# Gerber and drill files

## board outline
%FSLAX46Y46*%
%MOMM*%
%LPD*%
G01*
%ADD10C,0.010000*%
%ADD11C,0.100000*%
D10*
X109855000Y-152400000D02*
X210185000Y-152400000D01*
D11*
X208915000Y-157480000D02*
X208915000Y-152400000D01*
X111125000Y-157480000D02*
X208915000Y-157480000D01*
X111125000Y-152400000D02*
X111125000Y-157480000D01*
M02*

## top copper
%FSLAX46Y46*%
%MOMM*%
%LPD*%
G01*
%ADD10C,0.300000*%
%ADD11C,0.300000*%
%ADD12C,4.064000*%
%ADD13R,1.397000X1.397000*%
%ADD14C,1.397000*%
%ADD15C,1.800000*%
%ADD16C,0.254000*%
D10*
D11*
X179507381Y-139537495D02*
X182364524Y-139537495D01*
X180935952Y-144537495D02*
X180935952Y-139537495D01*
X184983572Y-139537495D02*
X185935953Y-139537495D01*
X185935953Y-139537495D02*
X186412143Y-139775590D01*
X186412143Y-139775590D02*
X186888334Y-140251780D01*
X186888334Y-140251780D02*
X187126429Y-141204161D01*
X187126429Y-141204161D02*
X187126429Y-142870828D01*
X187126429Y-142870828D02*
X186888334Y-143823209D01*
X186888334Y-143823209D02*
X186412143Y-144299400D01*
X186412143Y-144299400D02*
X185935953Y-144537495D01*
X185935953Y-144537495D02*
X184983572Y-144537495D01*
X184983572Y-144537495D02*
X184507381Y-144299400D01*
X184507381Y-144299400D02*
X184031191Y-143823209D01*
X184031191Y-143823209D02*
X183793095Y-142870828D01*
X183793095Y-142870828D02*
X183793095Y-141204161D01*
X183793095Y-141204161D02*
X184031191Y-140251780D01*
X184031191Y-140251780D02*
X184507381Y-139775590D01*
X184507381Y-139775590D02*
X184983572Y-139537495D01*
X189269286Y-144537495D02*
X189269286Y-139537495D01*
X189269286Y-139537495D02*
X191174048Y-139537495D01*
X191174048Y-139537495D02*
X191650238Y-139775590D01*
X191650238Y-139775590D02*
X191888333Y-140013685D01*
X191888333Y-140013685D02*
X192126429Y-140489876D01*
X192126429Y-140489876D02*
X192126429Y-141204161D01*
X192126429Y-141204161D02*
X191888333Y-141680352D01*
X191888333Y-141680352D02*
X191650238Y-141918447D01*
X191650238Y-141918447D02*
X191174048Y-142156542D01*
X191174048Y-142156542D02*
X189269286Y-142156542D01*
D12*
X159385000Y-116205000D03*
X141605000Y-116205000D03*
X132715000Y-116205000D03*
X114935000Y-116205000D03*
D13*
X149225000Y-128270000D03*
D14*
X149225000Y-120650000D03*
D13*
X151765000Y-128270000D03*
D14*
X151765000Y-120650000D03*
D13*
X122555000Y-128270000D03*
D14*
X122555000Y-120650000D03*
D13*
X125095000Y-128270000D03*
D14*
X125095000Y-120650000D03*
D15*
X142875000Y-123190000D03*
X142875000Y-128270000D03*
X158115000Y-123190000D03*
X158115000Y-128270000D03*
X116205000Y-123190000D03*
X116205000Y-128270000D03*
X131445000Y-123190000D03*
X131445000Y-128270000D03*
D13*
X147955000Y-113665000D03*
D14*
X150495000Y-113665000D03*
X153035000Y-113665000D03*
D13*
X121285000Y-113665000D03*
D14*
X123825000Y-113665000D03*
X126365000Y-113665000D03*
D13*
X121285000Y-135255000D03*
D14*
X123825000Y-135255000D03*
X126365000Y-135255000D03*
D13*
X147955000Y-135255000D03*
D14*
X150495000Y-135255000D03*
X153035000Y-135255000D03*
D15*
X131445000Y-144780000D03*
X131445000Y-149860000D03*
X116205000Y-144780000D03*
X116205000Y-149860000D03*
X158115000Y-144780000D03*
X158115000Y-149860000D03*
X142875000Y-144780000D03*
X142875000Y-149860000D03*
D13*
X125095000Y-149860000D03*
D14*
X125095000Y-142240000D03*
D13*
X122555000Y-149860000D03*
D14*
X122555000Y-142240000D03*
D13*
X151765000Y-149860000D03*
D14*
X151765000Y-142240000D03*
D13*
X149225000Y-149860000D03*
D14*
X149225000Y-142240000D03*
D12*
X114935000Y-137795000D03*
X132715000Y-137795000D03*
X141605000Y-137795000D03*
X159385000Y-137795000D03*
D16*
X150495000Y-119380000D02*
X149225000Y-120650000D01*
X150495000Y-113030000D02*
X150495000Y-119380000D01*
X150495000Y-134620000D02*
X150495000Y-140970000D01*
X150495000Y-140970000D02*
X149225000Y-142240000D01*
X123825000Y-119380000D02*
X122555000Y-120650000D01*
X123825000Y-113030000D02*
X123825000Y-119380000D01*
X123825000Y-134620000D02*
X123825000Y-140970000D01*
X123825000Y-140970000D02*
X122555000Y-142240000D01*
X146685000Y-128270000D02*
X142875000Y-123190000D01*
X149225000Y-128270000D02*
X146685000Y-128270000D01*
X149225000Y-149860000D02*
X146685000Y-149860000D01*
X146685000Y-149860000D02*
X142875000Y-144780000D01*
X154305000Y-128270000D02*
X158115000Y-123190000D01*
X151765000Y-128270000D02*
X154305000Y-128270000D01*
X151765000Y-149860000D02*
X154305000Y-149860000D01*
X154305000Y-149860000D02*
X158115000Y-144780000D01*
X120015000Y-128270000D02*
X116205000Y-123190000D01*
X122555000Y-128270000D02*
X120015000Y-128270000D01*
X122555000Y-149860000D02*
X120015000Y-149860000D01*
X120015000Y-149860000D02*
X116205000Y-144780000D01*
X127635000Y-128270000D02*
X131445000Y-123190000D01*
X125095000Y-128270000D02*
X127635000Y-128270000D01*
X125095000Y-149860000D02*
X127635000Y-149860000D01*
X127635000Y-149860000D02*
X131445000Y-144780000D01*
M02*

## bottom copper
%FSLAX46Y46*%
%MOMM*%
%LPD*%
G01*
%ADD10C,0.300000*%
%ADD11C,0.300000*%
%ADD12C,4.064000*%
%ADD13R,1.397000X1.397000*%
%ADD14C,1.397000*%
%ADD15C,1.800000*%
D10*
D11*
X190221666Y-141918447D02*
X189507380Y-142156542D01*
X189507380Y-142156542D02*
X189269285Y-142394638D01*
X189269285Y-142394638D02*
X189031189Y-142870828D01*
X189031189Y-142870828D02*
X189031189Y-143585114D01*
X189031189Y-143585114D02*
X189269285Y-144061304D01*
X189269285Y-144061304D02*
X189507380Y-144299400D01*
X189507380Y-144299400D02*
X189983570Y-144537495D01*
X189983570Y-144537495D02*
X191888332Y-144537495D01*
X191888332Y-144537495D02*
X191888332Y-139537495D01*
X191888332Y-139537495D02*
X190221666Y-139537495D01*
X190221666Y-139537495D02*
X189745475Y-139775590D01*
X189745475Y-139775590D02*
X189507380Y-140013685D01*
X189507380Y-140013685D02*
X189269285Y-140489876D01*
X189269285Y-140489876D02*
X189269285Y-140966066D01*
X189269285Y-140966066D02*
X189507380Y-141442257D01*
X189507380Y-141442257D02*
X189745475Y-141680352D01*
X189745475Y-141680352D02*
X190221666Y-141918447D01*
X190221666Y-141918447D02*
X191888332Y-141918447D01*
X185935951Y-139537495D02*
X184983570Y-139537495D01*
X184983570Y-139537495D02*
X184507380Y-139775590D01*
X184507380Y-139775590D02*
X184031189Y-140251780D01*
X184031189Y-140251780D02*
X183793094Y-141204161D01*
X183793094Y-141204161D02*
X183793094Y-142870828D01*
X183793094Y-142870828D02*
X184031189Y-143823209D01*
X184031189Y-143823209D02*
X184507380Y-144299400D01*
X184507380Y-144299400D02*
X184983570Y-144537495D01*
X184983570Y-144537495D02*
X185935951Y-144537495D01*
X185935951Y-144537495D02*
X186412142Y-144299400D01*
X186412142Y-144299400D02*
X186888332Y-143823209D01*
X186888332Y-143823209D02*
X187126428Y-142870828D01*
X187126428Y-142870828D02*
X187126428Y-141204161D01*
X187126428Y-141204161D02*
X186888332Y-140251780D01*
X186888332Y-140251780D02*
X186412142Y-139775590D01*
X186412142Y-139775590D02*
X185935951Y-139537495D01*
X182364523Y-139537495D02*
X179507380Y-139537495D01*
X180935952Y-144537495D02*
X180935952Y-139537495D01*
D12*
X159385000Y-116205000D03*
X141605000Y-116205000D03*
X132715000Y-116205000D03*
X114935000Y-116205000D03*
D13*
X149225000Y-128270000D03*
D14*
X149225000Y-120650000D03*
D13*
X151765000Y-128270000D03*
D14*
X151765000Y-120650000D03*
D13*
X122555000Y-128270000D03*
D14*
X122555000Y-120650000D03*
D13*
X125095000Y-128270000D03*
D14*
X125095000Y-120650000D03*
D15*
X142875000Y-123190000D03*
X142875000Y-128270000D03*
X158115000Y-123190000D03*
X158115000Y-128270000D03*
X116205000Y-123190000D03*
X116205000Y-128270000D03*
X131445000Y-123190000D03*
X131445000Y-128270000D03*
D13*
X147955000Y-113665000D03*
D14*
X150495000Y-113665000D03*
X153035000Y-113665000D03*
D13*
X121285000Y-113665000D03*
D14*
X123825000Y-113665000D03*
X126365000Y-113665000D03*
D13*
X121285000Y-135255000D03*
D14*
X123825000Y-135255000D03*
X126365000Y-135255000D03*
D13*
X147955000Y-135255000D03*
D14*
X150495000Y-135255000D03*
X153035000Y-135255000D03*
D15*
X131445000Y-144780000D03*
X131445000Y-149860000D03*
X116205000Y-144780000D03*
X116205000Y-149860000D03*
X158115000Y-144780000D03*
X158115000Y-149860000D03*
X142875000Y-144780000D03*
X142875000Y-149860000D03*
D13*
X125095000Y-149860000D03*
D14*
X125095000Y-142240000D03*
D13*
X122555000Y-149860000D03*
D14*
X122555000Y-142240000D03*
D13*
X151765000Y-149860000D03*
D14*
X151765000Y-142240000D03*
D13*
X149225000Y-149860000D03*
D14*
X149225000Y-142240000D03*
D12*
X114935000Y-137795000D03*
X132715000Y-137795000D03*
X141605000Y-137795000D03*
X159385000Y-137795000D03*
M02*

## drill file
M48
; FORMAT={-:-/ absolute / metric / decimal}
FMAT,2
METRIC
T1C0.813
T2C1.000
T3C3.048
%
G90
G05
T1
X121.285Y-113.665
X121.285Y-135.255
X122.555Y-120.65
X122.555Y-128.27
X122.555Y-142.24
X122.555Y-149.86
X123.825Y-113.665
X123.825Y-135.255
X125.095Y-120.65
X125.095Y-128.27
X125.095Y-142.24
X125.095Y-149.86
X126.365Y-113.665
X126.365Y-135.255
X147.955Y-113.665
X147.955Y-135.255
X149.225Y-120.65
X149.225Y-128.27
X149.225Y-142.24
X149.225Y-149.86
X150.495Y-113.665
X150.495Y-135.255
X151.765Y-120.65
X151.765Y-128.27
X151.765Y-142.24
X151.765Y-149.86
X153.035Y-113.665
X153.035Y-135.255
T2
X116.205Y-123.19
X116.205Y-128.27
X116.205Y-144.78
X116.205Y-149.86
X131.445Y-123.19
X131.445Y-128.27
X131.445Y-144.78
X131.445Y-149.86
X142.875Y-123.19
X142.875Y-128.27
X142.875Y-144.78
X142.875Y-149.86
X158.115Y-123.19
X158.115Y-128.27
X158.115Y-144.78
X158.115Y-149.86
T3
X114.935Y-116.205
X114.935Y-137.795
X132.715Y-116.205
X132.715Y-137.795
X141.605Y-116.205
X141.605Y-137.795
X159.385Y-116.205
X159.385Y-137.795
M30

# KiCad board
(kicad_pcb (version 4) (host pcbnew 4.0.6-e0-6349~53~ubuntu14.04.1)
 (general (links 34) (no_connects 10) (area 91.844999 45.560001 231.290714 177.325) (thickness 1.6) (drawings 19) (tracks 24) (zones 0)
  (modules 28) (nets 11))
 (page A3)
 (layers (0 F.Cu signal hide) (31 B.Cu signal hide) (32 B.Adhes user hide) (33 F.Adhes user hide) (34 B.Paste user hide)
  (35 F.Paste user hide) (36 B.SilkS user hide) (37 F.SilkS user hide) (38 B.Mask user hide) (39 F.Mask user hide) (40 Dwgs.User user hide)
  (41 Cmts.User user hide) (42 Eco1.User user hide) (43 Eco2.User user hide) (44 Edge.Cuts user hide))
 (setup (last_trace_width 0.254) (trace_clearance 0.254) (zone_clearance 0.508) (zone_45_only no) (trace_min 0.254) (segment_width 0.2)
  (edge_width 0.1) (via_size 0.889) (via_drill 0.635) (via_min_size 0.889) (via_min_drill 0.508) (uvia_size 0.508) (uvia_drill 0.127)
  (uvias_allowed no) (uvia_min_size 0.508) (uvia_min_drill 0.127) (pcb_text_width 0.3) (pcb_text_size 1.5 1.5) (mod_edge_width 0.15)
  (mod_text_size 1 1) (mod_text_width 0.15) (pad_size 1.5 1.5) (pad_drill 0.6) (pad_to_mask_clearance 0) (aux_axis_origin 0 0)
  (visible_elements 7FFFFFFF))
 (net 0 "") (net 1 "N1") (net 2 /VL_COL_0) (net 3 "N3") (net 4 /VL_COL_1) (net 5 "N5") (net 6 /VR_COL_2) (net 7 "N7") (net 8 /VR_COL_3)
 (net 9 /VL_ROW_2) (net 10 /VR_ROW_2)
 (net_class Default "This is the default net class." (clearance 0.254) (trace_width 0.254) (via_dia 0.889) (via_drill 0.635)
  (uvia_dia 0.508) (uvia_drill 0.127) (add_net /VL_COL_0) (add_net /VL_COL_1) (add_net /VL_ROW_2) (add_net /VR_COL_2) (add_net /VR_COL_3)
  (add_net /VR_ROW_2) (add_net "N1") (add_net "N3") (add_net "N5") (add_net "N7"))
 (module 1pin (layer F.Cu) (at 159.385 116.205)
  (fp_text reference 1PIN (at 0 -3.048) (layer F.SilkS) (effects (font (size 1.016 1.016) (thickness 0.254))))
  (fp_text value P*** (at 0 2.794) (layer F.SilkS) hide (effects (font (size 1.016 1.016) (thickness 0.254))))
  (pad 1 thru_hole circle (at 0 0) (size 4.064 4.064) (drill 3.048) (layers *.Cu *.Mask F.SilkS)))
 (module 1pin (layer F.Cu) (at 141.605 116.205)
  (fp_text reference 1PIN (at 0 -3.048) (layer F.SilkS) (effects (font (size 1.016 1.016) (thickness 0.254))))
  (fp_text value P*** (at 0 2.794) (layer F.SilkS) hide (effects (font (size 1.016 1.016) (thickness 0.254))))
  (pad 1 thru_hole circle (at 0 0) (size 4.064 4.064) (drill 3.048) (layers *.Cu *.Mask F.SilkS)))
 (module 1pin (layer F.Cu) (at 132.715 116.205)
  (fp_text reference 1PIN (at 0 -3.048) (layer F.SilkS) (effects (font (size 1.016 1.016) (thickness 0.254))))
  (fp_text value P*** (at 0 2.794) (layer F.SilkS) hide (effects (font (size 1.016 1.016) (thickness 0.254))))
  (pad 1 thru_hole circle (at 0 0) (size 4.064 4.064) (drill 3.048) (layers *.Cu *.Mask F.SilkS)))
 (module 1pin (layer F.Cu) (at 114.935 116.205)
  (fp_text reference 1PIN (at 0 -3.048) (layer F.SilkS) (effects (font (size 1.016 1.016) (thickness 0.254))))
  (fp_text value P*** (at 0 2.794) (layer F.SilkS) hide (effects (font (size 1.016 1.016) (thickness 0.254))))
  (pad 1 thru_hole circle (at 0 0) (size 4.064 4.064) (drill 3.048) (layers *.Cu *.Mask F.SilkS)))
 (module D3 (layer F.Cu) (at 149.225 124.46 270)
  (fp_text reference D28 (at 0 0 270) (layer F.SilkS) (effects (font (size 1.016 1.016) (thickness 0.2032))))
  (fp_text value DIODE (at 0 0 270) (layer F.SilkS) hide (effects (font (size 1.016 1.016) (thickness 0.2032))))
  (pad 2 thru_hole rect (at 3.81 0 270) (size 1.397 1.397) (drill 0.8128) (layers *.Cu *.Mask F.SilkS) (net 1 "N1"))
  (pad 1 thru_hole circle (at -3.81 0 270) (size 1.397 1.397) (drill 0.8128) (layers *.Cu *.Mask F.SilkS) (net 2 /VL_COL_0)))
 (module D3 (layer F.Cu) (at 151.765 124.46 270)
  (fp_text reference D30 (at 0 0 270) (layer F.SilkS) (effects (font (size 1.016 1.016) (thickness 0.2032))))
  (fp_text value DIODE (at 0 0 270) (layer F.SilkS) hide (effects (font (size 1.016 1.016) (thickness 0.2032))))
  (pad 2 thru_hole rect (at 3.81 0 270) (size 1.397 1.397) (drill 0.8128) (layers *.Cu *.Mask F.SilkS) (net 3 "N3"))
  (pad 1 thru_hole circle (at -3.81 0 270) (size 1.397 1.397) (drill 0.8128) (layers *.Cu *.Mask F.SilkS) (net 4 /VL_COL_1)))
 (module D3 (layer F.Cu) (at 122.555 124.46 270)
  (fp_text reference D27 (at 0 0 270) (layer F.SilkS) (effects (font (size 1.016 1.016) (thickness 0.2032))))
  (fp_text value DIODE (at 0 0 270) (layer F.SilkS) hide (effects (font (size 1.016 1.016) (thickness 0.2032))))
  (pad 2 thru_hole rect (at 3.81 0 270) (size 1.397 1.397) (drill 0.8128) (layers *.Cu *.Mask F.SilkS) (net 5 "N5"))
  (pad 1 thru_hole circle (at -3.81 0 270) (size 1.397 1.397) (drill 0.8128) (layers *.Cu *.Mask F.SilkS) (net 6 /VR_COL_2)))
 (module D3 (layer F.Cu) (at 125.095 124.46 270)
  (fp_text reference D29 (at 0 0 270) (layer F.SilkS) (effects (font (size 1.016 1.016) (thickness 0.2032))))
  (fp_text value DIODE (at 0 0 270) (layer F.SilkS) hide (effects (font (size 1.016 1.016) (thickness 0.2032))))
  (pad 2 thru_hole rect (at 3.81 0 270) (size 1.397 1.397) (drill 0.8128) (layers *.Cu *.Mask F.SilkS) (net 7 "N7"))
  (pad 1 thru_hole circle (at -3.81 0 270) (size 1.397 1.397) (drill 0.8128) (layers *.Cu *.Mask F.SilkS) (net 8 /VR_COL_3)))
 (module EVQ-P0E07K (layer F.Cu) (at 142.875 125.73)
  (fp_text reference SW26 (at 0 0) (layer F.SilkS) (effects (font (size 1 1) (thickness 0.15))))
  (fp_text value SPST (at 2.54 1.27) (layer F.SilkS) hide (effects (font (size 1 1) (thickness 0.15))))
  (pad 1 thru_hole circle (at 0 -2.54) (size 1.8 1.8) (drill 1) (layers *.Cu *.Mask F.SilkS) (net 1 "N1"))
  (pad 2 thru_hole circle (at 0 2.54) (size 1.8 1.8) (drill 1) (layers *.Cu *.Mask F.SilkS) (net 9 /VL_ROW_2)))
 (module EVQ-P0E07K (layer F.Cu) (at 158.115 125.73)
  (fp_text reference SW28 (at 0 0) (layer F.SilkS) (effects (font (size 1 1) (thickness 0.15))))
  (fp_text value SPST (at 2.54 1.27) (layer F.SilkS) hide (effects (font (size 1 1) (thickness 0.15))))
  (pad 1 thru_hole circle (at 0 -2.54) (size 1.8 1.8) (drill 1) (layers *.Cu *.Mask F.SilkS) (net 3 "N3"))
  (pad 2 thru_hole circle (at 0 2.54) (size 1.8 1.8) (drill 1) (layers *.Cu *.Mask F.SilkS) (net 9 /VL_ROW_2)))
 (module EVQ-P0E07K (layer F.Cu) (at 116.205 125.73)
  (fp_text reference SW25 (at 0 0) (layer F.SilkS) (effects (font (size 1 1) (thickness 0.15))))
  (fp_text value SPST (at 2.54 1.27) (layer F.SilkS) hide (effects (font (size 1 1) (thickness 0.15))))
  (pad 1 thru_hole circle (at 0 -2.54) (size 1.8 1.8) (drill 1) (layers *.Cu *.Mask F.SilkS) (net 5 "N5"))
  (pad 2 thru_hole circle (at 0 2.54) (size 1.8 1.8) (drill 1) (layers *.Cu *.Mask F.SilkS) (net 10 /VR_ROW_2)))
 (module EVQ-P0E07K (layer F.Cu) (at 131.445 125.73)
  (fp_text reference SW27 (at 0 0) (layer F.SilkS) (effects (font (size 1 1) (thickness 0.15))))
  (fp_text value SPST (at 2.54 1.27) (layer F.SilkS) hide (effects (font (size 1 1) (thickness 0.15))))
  (pad 1 thru_hole circle (at 0 -2.54) (size 1.8 1.8) (drill 1) (layers *.Cu *.Mask F.SilkS) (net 7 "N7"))
  (pad 2 thru_hole circle (at 0 2.54) (size 1.8 1.8) (drill 1) (layers *.Cu *.Mask F.SilkS) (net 10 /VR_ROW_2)))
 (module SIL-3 (layer F.Cu) (at 150.495 113.665)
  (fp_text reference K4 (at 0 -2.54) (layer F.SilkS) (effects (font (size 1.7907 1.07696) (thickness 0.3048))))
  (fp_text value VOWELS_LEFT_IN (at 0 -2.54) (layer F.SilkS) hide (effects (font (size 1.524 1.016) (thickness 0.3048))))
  (pad 1 thru_hole rect (at -2.54 0) (size 1.397 1.397) (drill 0.8128) (layers *.Cu *.Mask F.SilkS) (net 9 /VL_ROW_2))
  (pad 2 thru_hole circle (at 0 0) (size 1.397 1.397) (drill 0.8128) (layers *.Cu *.Mask F.SilkS) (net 2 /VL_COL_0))
  (pad 3 thru_hole circle (at 2.54 0) (size 1.397 1.397) (drill 0.8128) (layers *.Cu *.Mask F.SilkS) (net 4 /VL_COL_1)))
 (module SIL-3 (layer F.Cu) (at 123.825 113.665)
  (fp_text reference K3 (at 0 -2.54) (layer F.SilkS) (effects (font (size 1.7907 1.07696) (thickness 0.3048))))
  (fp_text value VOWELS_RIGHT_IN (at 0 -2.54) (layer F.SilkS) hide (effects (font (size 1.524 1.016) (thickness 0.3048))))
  (pad 1 thru_hole rect (at -2.54 0) (size 1.397 1.397) (drill 0.8128) (layers *.Cu *.Mask F.SilkS) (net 10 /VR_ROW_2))
  (pad 2 thru_hole circle (at 0 0) (size 1.397 1.397) (drill 0.8128) (layers *.Cu *.Mask F.SilkS) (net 6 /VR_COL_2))
  (pad 3 thru_hole circle (at 2.54 0) (size 1.397 1.397) (drill 0.8128) (layers *.Cu *.Mask F.SilkS) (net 8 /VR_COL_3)))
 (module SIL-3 (layer F.Cu) (at 123.825 135.255)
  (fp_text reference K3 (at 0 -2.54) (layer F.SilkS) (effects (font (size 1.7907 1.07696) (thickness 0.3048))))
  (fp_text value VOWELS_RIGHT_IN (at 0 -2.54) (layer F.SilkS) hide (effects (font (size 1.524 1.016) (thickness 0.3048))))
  (pad 1 thru_hole rect (at -2.54 0) (size 1.397 1.397) (drill 0.8128) (layers *.Cu *.Mask F.SilkS) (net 10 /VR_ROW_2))
  (pad 2 thru_hole circle (at 0 0) (size 1.397 1.397) (drill 0.8128) (layers *.Cu *.Mask F.SilkS) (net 6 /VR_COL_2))
  (pad 3 thru_hole circle (at 2.54 0) (size 1.397 1.397) (drill 0.8128) (layers *.Cu *.Mask F.SilkS) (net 8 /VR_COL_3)))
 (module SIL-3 (layer F.Cu) (at 150.495 135.255)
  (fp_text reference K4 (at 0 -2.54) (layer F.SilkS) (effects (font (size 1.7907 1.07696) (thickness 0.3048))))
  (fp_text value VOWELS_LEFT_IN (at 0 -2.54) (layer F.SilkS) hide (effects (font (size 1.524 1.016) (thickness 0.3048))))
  (pad 1 thru_hole rect (at -2.54 0) (size 1.397 1.397) (drill 0.8128) (layers *.Cu *.Mask F.SilkS) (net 9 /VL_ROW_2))
  (pad 2 thru_hole circle (at 0 0) (size 1.397 1.397) (drill 0.8128) (layers *.Cu *.Mask F.SilkS) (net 2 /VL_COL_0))
  (pad 3 thru_hole circle (at 2.54 0) (size 1.397 1.397) (drill 0.8128) (layers *.Cu *.Mask F.SilkS) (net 4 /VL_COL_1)))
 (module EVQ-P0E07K (layer F.Cu) (at 131.445 147.32)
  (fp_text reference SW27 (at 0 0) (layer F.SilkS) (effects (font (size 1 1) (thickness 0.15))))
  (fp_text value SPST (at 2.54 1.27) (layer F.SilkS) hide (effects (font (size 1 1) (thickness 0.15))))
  (pad 1 thru_hole circle (at 0 -2.54) (size 1.8 1.8) (drill 1) (layers *.Cu *.Mask F.SilkS) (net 7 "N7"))
  (pad 2 thru_hole circle (at 0 2.54) (size 1.8 1.8) (drill 1) (layers *.Cu *.Mask F.SilkS) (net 10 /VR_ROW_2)))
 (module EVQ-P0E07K (layer F.Cu) (at 116.205 147.32)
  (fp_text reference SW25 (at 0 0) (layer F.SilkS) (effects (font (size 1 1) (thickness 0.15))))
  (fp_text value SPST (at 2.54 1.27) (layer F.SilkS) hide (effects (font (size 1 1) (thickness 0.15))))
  (pad 1 thru_hole circle (at 0 -2.54) (size 1.8 1.8) (drill 1) (layers *.Cu *.Mask F.SilkS) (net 5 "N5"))
  (pad 2 thru_hole circle (at 0 2.54) (size 1.8 1.8) (drill 1) (layers *.Cu *.Mask F.SilkS) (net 10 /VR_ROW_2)))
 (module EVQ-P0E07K (layer F.Cu) (at 158.115 147.32)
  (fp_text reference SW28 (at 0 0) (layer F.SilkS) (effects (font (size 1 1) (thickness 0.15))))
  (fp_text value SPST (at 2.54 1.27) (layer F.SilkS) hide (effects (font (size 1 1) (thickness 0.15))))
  (pad 1 thru_hole circle (at 0 -2.54) (size 1.8 1.8) (drill 1) (layers *.Cu *.Mask F.SilkS) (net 3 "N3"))
  (pad 2 thru_hole circle (at 0 2.54) (size 1.8 1.8) (drill 1) (layers *.Cu *.Mask F.SilkS) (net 9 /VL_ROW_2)))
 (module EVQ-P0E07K (layer F.Cu) (at 142.875 147.32)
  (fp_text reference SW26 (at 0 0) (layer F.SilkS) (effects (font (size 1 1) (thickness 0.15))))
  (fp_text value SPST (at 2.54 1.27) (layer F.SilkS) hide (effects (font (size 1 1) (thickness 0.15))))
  (pad 1 thru_hole circle (at 0 -2.54) (size 1.8 1.8) (drill 1) (layers *.Cu *.Mask F.SilkS) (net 1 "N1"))
  (pad 2 thru_hole circle (at 0 2.54) (size 1.8 1.8) (drill 1) (layers *.Cu *.Mask F.SilkS) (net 9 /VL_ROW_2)))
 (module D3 (layer F.Cu) (at 125.095 146.05 270)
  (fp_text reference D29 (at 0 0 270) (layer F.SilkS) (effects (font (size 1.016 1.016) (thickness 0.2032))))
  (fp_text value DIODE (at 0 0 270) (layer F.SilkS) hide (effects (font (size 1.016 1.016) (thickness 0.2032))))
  (pad 2 thru_hole rect (at 3.81 0 270) (size 1.397 1.397) (drill 0.8128) (layers *.Cu *.Mask F.SilkS) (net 7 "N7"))
  (pad 1 thru_hole circle (at -3.81 0 270) (size 1.397 1.397) (drill 0.8128) (layers *.Cu *.Mask F.SilkS) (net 8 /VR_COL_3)))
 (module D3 (layer F.Cu) (at 122.555 146.05 270)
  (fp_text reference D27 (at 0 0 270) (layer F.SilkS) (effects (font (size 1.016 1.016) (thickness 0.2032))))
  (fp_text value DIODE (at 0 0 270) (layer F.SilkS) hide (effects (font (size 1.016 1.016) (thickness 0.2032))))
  (pad 2 thru_hole rect (at 3.81 0 270) (size 1.397 1.397) (drill 0.8128) (layers *.Cu *.Mask F.SilkS) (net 5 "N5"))
  (pad 1 thru_hole circle (at -3.81 0 270) (size 1.397 1.397) (drill 0.8128) (layers *.Cu *.Mask F.SilkS) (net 6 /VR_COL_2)))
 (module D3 (layer F.Cu) (at 151.765 146.05 270)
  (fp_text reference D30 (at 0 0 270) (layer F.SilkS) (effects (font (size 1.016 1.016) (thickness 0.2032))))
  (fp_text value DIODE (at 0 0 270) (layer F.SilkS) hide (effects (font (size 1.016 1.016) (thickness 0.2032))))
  (pad 2 thru_hole rect (at 3.81 0 270) (size 1.397 1.397) (drill 0.8128) (layers *.Cu *.Mask F.SilkS) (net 3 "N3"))
  (pad 1 thru_hole circle (at -3.81 0 270) (size 1.397 1.397) (drill 0.8128) (layers *.Cu *.Mask F.SilkS) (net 4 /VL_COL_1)))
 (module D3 (layer F.Cu) (at 149.225 146.05 270)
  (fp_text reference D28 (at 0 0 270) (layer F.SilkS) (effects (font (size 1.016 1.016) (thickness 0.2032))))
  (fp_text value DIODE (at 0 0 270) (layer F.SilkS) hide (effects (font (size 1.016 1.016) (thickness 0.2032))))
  (pad 2 thru_hole rect (at 3.81 0 270) (size 1.397 1.397) (drill 0.8128) (layers *.Cu *.Mask F.SilkS) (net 1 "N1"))
  (pad 1 thru_hole circle (at -3.81 0 270) (size 1.397 1.397) (drill 0.8128) (layers *.Cu *.Mask F.SilkS) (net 2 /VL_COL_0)))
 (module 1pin (layer F.Cu) (at 114.935 137.795)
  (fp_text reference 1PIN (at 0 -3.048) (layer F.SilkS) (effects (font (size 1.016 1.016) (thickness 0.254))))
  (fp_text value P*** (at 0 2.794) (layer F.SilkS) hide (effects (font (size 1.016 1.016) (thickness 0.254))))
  (pad 1 thru_hole circle (at 0 0) (size 4.064 4.064) (drill 3.048) (layers *.Cu *.Mask F.SilkS)))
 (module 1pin (layer F.Cu) (at 132.715 137.795)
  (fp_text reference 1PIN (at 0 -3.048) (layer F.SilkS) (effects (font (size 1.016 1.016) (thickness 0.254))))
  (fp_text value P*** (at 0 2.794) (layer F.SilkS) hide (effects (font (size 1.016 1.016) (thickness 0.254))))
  (pad 1 thru_hole circle (at 0 0) (size 4.064 4.064) (drill 3.048) (layers *.Cu *.Mask F.SilkS)))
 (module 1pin (layer F.Cu) (at 141.605 137.795)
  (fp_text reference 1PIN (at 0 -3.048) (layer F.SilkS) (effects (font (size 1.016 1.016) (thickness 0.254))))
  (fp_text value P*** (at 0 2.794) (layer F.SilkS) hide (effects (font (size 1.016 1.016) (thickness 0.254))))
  (pad 1 thru_hole circle (at 0 0) (size 4.064 4.064) (drill 3.048) (layers *.Cu *.Mask F.SilkS)))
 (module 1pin (layer F.Cu) (at 159.385 137.795)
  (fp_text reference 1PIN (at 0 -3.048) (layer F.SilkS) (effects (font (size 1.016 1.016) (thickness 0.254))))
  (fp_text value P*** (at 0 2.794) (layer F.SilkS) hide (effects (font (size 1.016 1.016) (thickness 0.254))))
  (pad 1 thru_hole circle (at 0 0) (size 4.064 4.064) (drill 3.048) (layers *.Cu *.Mask F.SilkS)))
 (gr_line (start 109.855 152.4) (end 210.185 152.4) (angle 90) (layer Edge.Cuts) (width 0.01))
 (gr_line (start 208.915 157.48) (end 208.915 152.4) (angle 90) (layer Edge.Cuts) (width 0.1))
 (gr_line (start 111.125 157.48) (end 208.915 157.48) (angle 90) (layer Edge.Cuts) (width 0.1))
 (gr_line (start 111.125 152.4) (end 111.125 157.48) (angle 90) (layer Edge.Cuts) (width 0.1))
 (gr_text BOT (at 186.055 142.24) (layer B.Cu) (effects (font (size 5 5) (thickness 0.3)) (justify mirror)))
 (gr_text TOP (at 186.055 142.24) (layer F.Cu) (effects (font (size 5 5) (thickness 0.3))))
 (segment (start 150.495 119.38) (end 149.225 120.65) (width 0.254) (layer F.Cu) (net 2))
 (segment (start 150.495 113.03) (end 150.495 119.38) (width 0.254) (layer F.Cu) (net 2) (status 10))
 (segment (start 150.495 134.62) (end 150.495 140.97) (width 0.254) (layer F.Cu) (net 2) (status 10))
 (segment (start 150.495 140.97) (end 149.225 142.24) (width 0.254) (layer F.Cu) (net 2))
 (segment (start 123.825 119.38) (end 122.555 120.65) (width 0.254) (layer F.Cu) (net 6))
 (segment (start 123.825 113.03) (end 123.825 119.38) (width 0.254) (layer F.Cu) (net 6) (status 10))
 (segment (start 123.825 134.62) (end 123.825 140.97) (width 0.254) (layer F.Cu) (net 6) (status 10))
 (segment (start 123.825 140.97) (end 122.555 142.24) (width 0.254) (layer F.Cu) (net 6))
 (segment (start 146.685 128.27) (end 142.875 123.19) (width 0.254) (layer F.Cu) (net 1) (status 20))
 (segment (start 149.225 128.27) (end 146.685 128.27) (width 0.254) (layer F.Cu) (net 1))
 (segment (start 149.225 149.86) (end 146.685 149.86) (width 0.254) (layer F.Cu) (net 1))
 (segment (start 146.685 149.86) (end 142.875 144.78) (width 0.254) (layer F.Cu) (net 1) (status 20))
 (segment (start 154.305 128.27) (end 158.115 123.19) (width 0.254) (layer F.Cu) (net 3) (status 20))
 (segment (start 151.765 128.27) (end 154.305 128.27) (width 0.254) (layer F.Cu) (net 3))
 (segment (start 151.765 149.86) (end 154.305 149.86) (width 0.254) (layer F.Cu) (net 3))
 (segment (start 154.305 149.86) (end 158.115 144.78) (width 0.254) (layer F.Cu) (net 3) (status 20))
 (segment (start 120.015 128.27) (end 116.205 123.19) (width 0.254) (layer F.Cu) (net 5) (status 20))
 (segment (start 122.555 128.27) (end 120.015 128.27) (width 0.254) (layer F.Cu) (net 5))
 (segment (start 122.555 149.86) (end 120.015 149.86) (width 0.254) (layer F.Cu) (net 5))
 (segment (start 120.015 149.86) (end 116.205 144.78) (width 0.254) (layer F.Cu) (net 5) (status 20))
 (segment (start 127.635 128.27) (end 131.445 123.19) (width 0.254) (layer F.Cu) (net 7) (status 20))
 (segment (start 125.095 128.27) (end 127.635 128.27) (width 0.254) (layer F.Cu) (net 7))
 (segment (start 125.095 149.86) (end 127.635 149.86) (width 0.254) (layer F.Cu) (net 7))
 (segment (start 127.635 149.86) (end 131.445 144.78) (width 0.254) (layer F.Cu) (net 7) (status 20))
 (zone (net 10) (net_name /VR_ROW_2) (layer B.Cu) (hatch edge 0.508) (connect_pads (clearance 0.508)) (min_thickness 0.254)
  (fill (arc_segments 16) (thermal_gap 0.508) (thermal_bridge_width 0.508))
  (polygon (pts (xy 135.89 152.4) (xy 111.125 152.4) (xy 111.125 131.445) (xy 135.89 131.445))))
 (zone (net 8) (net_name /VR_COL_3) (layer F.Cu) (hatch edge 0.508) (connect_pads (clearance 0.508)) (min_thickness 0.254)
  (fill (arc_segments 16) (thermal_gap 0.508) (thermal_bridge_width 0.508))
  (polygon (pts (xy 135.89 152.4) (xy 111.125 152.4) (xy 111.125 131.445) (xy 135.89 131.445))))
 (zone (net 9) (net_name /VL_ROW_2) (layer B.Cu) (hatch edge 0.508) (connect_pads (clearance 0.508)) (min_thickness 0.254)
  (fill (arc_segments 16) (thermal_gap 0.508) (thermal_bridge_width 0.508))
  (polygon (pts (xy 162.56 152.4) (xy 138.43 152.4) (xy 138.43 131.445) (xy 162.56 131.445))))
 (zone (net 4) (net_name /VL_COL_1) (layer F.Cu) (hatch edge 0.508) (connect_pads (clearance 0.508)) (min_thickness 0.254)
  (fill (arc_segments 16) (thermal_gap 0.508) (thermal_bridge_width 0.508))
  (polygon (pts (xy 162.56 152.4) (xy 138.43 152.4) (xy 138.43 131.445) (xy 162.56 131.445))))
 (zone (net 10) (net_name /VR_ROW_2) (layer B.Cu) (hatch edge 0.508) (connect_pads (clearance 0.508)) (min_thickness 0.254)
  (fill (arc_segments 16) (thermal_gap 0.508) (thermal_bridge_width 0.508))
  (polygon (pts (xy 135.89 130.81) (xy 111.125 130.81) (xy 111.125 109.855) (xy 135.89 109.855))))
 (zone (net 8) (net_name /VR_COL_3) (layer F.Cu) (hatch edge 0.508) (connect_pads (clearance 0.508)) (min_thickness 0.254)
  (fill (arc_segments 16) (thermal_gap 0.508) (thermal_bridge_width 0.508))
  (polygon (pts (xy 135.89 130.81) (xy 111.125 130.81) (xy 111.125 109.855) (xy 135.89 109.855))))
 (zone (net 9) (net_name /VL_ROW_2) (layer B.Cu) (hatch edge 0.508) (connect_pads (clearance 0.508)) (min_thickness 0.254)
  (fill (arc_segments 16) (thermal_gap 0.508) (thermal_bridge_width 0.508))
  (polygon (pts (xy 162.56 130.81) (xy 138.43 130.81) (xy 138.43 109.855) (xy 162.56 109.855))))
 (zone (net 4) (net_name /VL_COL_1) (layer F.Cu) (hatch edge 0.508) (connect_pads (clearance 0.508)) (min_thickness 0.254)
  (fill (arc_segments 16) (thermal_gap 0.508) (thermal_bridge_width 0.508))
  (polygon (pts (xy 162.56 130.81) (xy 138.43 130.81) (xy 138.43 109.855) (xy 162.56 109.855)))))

